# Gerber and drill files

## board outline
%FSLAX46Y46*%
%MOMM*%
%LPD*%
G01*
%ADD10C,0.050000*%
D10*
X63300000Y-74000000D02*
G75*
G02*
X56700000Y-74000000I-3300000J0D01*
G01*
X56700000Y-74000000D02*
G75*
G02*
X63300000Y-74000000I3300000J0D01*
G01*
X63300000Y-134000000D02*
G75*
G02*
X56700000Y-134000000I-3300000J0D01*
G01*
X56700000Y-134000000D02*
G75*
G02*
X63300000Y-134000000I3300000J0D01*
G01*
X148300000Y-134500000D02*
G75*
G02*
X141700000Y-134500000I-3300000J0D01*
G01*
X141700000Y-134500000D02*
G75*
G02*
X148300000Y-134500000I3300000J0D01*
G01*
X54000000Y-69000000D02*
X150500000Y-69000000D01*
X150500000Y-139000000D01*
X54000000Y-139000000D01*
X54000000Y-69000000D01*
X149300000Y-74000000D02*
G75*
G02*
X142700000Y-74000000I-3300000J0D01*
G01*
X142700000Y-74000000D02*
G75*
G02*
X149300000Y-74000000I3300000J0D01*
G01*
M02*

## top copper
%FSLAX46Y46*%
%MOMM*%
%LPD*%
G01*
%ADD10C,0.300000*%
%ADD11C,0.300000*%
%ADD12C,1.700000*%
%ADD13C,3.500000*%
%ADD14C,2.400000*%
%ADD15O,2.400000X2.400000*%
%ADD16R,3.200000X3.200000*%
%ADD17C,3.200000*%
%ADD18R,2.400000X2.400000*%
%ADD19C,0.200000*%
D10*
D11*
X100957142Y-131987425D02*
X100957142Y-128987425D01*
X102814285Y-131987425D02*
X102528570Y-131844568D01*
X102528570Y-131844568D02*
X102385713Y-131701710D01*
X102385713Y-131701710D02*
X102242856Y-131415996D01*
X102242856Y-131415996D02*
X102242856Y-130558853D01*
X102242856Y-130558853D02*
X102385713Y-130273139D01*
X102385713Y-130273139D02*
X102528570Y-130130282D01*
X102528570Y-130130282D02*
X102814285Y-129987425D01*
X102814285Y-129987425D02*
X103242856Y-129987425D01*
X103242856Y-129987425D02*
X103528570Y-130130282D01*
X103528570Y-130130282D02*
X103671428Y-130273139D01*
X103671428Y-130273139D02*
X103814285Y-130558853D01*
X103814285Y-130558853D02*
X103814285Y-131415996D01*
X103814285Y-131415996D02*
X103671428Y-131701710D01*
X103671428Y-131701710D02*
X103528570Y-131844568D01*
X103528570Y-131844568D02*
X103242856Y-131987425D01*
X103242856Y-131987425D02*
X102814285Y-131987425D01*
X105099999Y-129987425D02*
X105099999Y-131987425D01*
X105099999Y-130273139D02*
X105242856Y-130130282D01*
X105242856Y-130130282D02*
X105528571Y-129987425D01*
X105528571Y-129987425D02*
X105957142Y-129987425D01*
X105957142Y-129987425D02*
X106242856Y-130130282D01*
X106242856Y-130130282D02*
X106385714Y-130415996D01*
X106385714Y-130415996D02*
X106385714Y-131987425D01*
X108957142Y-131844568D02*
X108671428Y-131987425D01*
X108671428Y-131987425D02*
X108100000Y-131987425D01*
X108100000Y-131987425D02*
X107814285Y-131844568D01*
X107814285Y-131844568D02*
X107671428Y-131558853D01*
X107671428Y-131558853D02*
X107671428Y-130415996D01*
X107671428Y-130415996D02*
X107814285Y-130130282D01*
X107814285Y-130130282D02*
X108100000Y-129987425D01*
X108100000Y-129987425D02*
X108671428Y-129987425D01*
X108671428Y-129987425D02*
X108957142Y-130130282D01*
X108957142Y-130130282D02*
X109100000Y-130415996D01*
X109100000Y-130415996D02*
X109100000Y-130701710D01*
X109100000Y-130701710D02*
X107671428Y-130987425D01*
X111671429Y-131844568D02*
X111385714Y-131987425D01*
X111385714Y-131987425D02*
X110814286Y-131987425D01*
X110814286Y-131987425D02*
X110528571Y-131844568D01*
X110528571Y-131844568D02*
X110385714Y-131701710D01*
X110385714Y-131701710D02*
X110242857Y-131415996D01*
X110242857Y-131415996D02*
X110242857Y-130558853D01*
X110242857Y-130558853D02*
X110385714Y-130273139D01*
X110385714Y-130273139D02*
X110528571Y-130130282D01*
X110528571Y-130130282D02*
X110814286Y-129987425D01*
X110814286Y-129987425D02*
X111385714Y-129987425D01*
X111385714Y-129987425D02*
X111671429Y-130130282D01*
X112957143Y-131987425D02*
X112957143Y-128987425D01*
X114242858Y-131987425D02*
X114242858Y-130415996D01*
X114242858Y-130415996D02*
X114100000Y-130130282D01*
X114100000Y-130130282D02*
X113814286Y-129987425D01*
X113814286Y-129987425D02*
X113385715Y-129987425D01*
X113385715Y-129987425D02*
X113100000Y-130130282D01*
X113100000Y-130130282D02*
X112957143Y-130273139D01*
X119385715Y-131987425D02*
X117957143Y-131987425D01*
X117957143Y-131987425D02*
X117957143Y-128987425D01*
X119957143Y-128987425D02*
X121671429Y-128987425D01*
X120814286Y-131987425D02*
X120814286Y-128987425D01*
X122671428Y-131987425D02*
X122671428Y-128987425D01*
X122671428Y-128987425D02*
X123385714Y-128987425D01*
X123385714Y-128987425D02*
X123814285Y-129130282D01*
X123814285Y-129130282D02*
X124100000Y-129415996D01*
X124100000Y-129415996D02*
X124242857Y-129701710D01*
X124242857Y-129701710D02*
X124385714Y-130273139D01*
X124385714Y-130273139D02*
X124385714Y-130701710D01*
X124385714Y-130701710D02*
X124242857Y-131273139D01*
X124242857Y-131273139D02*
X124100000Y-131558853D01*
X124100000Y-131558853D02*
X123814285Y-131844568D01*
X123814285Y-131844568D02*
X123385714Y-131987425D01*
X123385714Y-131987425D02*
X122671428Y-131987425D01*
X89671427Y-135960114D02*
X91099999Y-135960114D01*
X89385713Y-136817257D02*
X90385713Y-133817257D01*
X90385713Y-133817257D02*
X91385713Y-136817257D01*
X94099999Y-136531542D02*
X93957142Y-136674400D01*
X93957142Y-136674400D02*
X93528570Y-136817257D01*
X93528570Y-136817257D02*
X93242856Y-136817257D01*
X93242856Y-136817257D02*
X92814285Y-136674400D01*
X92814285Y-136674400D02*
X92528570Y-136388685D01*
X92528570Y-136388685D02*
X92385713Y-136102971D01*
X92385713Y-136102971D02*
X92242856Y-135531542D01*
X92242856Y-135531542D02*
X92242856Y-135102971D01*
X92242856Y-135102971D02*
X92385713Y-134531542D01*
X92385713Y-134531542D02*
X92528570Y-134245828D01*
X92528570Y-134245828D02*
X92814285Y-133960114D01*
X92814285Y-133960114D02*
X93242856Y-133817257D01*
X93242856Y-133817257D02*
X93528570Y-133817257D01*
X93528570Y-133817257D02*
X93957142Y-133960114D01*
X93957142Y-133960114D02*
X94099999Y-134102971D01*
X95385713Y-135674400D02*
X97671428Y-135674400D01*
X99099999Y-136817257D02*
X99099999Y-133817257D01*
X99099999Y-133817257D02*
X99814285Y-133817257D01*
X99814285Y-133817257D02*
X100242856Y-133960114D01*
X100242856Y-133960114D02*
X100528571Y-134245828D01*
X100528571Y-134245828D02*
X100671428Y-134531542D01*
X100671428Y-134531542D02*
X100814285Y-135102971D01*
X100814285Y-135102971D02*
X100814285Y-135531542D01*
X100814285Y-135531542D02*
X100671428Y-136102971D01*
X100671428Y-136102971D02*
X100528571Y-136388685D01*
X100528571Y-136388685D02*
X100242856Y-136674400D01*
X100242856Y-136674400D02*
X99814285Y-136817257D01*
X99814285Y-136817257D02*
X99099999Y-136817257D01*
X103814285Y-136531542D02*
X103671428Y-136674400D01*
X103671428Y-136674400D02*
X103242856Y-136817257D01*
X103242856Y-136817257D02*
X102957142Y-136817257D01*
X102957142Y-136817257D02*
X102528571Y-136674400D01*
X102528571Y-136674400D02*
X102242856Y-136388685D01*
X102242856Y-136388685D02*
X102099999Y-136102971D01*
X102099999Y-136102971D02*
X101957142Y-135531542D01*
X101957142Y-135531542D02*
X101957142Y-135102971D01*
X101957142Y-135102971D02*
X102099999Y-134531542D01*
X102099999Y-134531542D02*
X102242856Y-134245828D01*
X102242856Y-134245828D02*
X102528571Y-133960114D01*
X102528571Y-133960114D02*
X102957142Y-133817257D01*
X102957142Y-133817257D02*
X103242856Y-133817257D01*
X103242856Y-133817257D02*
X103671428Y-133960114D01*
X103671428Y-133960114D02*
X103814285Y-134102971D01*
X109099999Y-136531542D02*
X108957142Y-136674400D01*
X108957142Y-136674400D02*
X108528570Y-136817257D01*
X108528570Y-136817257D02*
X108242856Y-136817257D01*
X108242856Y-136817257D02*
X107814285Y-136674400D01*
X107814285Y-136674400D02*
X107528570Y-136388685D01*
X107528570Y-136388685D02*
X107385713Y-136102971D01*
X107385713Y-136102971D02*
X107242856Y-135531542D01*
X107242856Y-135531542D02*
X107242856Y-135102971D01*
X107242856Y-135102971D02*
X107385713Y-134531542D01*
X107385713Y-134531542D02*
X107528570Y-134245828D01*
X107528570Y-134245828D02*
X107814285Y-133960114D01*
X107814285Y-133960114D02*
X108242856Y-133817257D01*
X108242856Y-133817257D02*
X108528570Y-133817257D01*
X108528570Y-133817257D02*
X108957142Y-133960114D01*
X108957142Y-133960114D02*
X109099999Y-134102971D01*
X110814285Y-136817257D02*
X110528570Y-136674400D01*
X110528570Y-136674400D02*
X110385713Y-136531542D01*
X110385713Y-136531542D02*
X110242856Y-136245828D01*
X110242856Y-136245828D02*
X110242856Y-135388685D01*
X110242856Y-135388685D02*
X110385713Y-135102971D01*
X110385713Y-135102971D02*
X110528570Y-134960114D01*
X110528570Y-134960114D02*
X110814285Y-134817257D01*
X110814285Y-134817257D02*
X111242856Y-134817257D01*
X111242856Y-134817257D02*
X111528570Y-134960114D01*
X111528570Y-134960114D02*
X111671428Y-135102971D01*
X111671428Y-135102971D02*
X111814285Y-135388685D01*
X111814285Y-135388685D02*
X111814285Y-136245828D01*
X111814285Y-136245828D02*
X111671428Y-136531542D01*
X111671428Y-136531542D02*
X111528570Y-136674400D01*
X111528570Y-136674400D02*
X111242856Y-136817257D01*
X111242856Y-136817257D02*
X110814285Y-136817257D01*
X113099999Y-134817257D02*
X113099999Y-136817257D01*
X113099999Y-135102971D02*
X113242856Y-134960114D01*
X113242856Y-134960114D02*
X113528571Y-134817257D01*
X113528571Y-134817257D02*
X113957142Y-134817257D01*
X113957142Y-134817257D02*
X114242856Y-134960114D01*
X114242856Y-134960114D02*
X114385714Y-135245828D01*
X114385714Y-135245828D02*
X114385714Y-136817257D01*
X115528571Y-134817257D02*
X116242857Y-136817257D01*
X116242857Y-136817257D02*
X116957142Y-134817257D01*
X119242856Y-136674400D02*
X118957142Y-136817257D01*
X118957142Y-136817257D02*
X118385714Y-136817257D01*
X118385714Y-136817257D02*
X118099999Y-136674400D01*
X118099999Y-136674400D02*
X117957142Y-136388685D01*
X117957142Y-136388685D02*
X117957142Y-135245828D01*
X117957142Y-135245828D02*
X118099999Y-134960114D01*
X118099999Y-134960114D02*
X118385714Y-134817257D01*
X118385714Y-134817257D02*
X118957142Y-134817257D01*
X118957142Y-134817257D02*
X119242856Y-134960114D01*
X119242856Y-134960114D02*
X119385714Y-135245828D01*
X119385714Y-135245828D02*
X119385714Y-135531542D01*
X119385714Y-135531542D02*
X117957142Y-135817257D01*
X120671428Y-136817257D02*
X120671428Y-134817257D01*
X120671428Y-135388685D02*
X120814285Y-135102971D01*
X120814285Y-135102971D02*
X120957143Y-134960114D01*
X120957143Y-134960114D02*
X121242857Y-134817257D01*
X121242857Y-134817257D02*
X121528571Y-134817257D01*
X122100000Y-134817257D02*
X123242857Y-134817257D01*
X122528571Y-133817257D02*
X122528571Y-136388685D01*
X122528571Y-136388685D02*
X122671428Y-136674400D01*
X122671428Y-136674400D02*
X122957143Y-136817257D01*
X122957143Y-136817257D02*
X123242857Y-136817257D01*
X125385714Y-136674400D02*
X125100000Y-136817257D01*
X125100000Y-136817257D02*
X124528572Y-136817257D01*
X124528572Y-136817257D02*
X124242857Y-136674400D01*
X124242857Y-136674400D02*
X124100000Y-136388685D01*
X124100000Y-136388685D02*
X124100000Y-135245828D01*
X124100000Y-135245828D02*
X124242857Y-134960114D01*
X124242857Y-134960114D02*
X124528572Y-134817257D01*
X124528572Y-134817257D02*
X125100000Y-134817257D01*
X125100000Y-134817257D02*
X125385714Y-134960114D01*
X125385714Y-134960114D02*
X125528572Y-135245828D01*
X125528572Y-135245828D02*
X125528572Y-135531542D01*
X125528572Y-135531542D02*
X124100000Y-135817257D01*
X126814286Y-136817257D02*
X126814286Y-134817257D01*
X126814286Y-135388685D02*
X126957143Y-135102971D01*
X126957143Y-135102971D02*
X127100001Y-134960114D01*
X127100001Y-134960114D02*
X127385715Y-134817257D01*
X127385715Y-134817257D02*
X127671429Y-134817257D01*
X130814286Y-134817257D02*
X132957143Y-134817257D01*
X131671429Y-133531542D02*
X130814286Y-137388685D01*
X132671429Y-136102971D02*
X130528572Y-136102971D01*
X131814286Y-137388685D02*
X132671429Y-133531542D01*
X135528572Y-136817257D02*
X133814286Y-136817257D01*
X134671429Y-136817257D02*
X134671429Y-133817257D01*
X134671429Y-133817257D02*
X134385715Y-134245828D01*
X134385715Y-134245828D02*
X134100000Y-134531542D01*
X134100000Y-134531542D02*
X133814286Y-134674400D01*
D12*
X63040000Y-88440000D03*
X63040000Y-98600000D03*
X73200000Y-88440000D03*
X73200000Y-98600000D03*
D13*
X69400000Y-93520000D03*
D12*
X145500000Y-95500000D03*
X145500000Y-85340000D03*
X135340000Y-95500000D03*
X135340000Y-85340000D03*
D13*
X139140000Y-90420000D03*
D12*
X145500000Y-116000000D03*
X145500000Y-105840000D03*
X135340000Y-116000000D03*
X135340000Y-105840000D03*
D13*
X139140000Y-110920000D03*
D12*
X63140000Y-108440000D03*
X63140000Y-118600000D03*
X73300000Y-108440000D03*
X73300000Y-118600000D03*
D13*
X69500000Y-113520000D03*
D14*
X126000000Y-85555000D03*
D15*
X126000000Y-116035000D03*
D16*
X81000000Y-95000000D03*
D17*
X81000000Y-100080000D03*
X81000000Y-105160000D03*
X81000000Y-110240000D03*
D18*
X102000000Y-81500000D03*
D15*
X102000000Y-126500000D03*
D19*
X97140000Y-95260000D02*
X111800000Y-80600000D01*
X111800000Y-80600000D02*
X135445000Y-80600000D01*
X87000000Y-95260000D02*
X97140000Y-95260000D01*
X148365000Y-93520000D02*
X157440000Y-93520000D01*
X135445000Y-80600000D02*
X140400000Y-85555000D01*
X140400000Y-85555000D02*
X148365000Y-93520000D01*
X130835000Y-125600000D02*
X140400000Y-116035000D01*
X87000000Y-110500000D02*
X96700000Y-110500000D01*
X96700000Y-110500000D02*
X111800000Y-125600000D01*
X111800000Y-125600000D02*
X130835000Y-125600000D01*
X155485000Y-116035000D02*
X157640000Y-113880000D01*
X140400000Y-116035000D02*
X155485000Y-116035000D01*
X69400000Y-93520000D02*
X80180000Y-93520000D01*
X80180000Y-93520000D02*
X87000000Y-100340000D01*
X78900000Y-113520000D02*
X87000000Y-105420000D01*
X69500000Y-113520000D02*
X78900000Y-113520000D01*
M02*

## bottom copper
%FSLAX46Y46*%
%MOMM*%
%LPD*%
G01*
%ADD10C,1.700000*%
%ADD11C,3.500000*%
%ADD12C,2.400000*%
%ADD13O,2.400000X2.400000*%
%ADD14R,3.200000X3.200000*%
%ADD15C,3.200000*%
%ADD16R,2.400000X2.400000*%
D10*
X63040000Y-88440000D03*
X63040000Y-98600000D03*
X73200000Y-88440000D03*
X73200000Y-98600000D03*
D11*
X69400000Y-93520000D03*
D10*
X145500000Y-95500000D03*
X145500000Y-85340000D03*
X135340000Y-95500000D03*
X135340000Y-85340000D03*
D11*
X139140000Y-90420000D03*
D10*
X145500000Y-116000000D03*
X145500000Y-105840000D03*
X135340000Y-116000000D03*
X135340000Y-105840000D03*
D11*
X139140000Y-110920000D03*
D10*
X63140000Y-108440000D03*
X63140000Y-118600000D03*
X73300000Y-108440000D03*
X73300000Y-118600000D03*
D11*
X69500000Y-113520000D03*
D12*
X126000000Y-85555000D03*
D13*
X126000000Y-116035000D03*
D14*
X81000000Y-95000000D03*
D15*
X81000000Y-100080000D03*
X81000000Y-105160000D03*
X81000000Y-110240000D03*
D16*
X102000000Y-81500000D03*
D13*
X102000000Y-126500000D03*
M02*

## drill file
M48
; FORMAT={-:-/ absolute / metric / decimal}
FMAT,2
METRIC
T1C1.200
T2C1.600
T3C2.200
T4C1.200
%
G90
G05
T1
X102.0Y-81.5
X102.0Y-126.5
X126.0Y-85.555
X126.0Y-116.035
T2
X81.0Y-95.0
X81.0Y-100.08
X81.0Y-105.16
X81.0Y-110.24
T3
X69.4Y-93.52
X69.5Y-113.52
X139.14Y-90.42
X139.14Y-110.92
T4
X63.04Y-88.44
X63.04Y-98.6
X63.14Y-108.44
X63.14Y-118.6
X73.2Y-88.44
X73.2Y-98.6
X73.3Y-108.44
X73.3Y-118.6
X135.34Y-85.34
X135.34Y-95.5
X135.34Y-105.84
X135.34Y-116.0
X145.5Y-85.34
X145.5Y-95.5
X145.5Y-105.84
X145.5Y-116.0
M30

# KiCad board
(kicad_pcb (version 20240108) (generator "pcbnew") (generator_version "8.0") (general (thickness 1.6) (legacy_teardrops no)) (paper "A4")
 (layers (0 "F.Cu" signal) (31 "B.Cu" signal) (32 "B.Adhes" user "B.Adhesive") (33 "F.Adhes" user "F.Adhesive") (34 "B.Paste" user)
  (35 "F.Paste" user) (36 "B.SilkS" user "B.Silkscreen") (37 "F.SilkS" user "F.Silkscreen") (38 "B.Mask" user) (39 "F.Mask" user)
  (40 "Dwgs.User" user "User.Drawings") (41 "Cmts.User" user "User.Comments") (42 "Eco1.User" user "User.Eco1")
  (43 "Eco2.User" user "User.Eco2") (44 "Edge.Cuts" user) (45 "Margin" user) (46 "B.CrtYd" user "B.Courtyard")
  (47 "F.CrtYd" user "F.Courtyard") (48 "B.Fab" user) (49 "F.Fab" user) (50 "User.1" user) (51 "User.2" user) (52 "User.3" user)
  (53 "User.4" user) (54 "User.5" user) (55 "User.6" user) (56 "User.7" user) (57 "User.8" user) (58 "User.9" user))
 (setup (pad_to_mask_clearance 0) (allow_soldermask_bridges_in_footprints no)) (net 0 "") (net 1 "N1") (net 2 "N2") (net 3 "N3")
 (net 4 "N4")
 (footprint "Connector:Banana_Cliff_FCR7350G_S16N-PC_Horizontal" (layer "F.Cu") (at 69.4 93.52)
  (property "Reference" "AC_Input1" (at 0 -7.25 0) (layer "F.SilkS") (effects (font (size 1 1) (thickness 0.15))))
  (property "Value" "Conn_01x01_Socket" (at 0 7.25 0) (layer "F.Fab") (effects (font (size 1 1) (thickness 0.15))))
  (pad "" np_thru_hole circle (at -6.36 -5.08) (size 1.7 1.7) (drill 1.2) (layers "F&B.Cu" "*.Mask"))
  (pad "" np_thru_hole circle (at -6.36 5.08) (size 1.7 1.7) (drill 1.2) (layers "F&B.Cu" "*.Mask"))
  (pad "" np_thru_hole circle (at 3.8 -5.08) (size 1.7 1.7) (drill 1.2) (layers "F&B.Cu" "*.Mask"))
  (pad "" np_thru_hole circle (at 3.8 5.08) (size 1.7 1.7) (drill 1.2) (layers "F&B.Cu" "*.Mask"))
  (pad "1" thru_hole circle (at 0 0) (size 3.5 3.5) (drill 2.2) (layers "*.Cu" "*.Mask") (remove_unused_layers no) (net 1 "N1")))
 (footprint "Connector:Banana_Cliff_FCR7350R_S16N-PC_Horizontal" (layer "F.Cu") (at 139.14 90.42 180)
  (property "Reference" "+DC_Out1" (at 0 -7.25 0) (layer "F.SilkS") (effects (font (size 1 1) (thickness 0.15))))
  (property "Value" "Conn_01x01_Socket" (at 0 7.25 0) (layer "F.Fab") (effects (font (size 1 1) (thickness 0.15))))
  (pad "" np_thru_hole circle (at -6.36 -5.08 180) (size 1.7 1.7) (drill 1.2) (layers "F&B.Cu" "*.Mask"))
  (pad "" np_thru_hole circle (at -6.36 5.08 180) (size 1.7 1.7) (drill 1.2) (layers "F&B.Cu" "*.Mask"))
  (pad "" np_thru_hole circle (at 3.8 -5.08 180) (size 1.7 1.7) (drill 1.2) (layers "F&B.Cu" "*.Mask"))
  (pad "" np_thru_hole circle (at 3.8 5.08 180) (size 1.7 1.7) (drill 1.2) (layers "F&B.Cu" "*.Mask"))
  (pad "1" thru_hole circle (at 0 0 180) (size 3.5 3.5) (drill 2.2) (layers "*.Cu" "*.Mask") (remove_unused_layers no) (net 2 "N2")))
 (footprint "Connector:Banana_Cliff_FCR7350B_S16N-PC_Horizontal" (layer "F.Cu") (at 139.14 110.92 180)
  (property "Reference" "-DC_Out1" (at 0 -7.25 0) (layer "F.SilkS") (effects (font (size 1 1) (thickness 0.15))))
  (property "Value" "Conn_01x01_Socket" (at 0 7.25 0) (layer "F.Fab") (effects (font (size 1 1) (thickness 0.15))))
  (pad "" np_thru_hole circle (at -6.36 -5.08 180) (size 1.7 1.7) (drill 1.2) (layers "F&B.Cu" "*.Mask"))
  (pad "" np_thru_hole circle (at -6.36 5.08 180) (size 1.7 1.7) (drill 1.2) (layers "F&B.Cu" "*.Mask"))
  (pad "" np_thru_hole circle (at 3.8 -5.08 180) (size 1.7 1.7) (drill 1.2) (layers "F&B.Cu" "*.Mask"))
  (pad "" np_thru_hole circle (at 3.8 5.08 180) (size 1.7 1.7) (drill 1.2) (layers "F&B.Cu" "*.Mask"))
  (pad "1" thru_hole circle (at 0 0 180) (size 3.5 3.5) (drill 2.2) (layers "*.Cu" "*.Mask") (remove_unused_layers no) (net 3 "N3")))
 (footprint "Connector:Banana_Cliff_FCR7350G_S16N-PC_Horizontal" (layer "F.Cu") (at 69.5 113.52)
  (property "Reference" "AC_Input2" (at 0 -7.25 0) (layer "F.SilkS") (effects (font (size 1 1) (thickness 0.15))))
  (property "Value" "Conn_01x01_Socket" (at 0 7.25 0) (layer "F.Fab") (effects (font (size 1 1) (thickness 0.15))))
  (pad "" np_thru_hole circle (at -6.36 -5.08) (size 1.7 1.7) (drill 1.2) (layers "F&B.Cu" "*.Mask"))
  (pad "" np_thru_hole circle (at -6.36 5.08) (size 1.7 1.7) (drill 1.2) (layers "F&B.Cu" "*.Mask"))
  (pad "" np_thru_hole circle (at 3.8 -5.08) (size 1.7 1.7) (drill 1.2) (layers "F&B.Cu" "*.Mask"))
  (pad "" np_thru_hole circle (at 3.8 5.08) (size 1.7 1.7) (drill 1.2) (layers "F&B.Cu" "*.Mask"))
  (pad "1" thru_hole circle (at 0 0) (size 3.5 3.5) (drill 2.2) (layers "*.Cu" "*.Mask") (remove_unused_layers no) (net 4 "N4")))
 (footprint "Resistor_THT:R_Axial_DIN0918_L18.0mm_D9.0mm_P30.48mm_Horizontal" (layer "F.Cu") (at 126 85.555 -90)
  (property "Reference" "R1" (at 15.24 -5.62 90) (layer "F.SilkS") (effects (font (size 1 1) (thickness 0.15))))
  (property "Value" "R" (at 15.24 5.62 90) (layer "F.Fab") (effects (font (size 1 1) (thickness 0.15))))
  (pad "1" thru_hole circle (at 0 0 270) (size 2.4 2.4) (drill 1.2) (layers "*.Cu" "*.Mask") (remove_unused_layers no) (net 2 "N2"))
  (pad "2" thru_hole oval (at 30.48 0 270) (size 2.4 2.4) (drill 1.2) (layers "*.Cu" "*.Mask") (remove_unused_layers no) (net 3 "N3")))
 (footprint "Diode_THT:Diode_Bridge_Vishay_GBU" (layer "F.Cu") (at 81 95 -90)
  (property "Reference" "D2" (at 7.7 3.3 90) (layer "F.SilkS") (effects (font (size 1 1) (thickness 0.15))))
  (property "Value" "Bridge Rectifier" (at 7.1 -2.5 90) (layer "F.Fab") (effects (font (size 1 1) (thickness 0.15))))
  (pad "1" thru_hole rect (at 0 0 270) (size 3.2 3.2) (drill 1.6) (layers "*.Cu" "*.Mask") (remove_unused_layers no) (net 2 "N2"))
  (pad "2" thru_hole circle (at 5.08 0 270) (size 3.2 3.2) (drill 1.6) (layers "*.Cu" "*.Mask") (remove_unused_layers no) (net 1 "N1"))
  (pad "3" thru_hole circle (at 10.16 0 270) (size 3.2 3.2) (drill 1.6) (layers "*.Cu" "*.Mask") (remove_unused_layers no) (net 4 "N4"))
  (pad "4" thru_hole circle (at 15.24 0 270) (size 3.2 3.2) (drill 1.6) (layers "*.Cu" "*.Mask") (remove_unused_layers no) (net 3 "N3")))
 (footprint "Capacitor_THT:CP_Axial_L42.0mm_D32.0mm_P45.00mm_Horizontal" (layer "F.Cu") (at 102 81.5 -90)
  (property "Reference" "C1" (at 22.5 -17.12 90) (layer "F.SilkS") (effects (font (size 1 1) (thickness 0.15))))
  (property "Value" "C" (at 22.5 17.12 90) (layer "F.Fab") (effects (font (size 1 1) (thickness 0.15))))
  (pad "1" thru_hole rect (at 0 0 270) (size 2.4 2.4) (drill 1.2) (layers "*.Cu" "*.Mask") (remove_unused_layers no) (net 2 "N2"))
  (pad "2" thru_hole oval (at 45 0 270) (size 2.4 2.4) (drill 1.2) (layers "*.Cu" "*.Mask") (remove_unused_layers no) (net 3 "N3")))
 (gr_circle (center 60 74) (end 63.3 74) (stroke (width 0.05) (type default)) (fill none) (layer "Edge.Cuts"))
 (gr_circle (center 60 134) (end 63.3 134) (stroke (width 0.05) (type default)) (fill none) (layer "Edge.Cuts"))
 (gr_circle (center 145 134.5) (end 148.3 134.5) (stroke (width 0.05) (type default)) (fill none) (layer "Edge.Cuts"))
 (gr_rect (start 54 69) (end 150.5 139) (stroke (width 0.05) (type default)) (fill none) (layer "Edge.Cuts"))
 (gr_circle (center 146 74) (end 149.3 74) (stroke (width 0.05) (type default)) (fill none) (layer "Edge.Cuts"))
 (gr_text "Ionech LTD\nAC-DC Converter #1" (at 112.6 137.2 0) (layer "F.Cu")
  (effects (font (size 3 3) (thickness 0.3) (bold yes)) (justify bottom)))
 (segment (start 97.14 95.26) (end 111.8 80.6) (width 0.2) (layer "F.Cu") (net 2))
 (segment (start 111.8 80.6) (end 135.445 80.6) (width 0.2) (layer "F.Cu") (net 2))
 (segment (start 87 95.26) (end 97.14 95.26) (width 0.2) (layer "F.Cu") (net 2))
 (segment (start 148.365 93.52) (end 157.44 93.52) (width 0.2) (layer "F.Cu") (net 2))
 (segment (start 135.445 80.6) (end 140.4 85.555) (width 0.2) (layer "F.Cu") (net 2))
 (segment (start 140.4 85.555) (end 148.365 93.52) (width 0.2) (layer "F.Cu") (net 2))
 (segment (start 130.835 125.6) (end 140.4 116.035) (width 0.2) (layer "F.Cu") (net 3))
 (segment (start 87 110.5) (end 96.7 110.5) (width 0.2) (layer "F.Cu") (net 3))
 (segment (start 96.7 110.5) (end 111.8 125.6) (width 0.2) (layer "F.Cu") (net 3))
 (segment (start 111.8 125.6) (end 130.835 125.6) (width 0.2) (layer "F.Cu") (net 3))
 (segment (start 155.485 116.035) (end 157.64 113.88) (width 0.2) (layer "F.Cu") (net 3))
 (segment (start 140.4 116.035) (end 155.485 116.035) (width 0.2) (layer "F.Cu") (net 3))
 (segment (start 69.4 93.52) (end 80.18 93.52) (width 0.2) (layer "F.Cu") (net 1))
 (segment (start 80.18 93.52) (end 87 100.34) (width 0.2) (layer "F.Cu") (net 1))
 (segment (start 78.9 113.52) (end 87 105.42) (width 0.2) (layer "F.Cu") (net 4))
 (segment (start 69.5 113.52) (end 78.9 113.52) (width 0.2) (layer "F.Cu") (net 4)))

